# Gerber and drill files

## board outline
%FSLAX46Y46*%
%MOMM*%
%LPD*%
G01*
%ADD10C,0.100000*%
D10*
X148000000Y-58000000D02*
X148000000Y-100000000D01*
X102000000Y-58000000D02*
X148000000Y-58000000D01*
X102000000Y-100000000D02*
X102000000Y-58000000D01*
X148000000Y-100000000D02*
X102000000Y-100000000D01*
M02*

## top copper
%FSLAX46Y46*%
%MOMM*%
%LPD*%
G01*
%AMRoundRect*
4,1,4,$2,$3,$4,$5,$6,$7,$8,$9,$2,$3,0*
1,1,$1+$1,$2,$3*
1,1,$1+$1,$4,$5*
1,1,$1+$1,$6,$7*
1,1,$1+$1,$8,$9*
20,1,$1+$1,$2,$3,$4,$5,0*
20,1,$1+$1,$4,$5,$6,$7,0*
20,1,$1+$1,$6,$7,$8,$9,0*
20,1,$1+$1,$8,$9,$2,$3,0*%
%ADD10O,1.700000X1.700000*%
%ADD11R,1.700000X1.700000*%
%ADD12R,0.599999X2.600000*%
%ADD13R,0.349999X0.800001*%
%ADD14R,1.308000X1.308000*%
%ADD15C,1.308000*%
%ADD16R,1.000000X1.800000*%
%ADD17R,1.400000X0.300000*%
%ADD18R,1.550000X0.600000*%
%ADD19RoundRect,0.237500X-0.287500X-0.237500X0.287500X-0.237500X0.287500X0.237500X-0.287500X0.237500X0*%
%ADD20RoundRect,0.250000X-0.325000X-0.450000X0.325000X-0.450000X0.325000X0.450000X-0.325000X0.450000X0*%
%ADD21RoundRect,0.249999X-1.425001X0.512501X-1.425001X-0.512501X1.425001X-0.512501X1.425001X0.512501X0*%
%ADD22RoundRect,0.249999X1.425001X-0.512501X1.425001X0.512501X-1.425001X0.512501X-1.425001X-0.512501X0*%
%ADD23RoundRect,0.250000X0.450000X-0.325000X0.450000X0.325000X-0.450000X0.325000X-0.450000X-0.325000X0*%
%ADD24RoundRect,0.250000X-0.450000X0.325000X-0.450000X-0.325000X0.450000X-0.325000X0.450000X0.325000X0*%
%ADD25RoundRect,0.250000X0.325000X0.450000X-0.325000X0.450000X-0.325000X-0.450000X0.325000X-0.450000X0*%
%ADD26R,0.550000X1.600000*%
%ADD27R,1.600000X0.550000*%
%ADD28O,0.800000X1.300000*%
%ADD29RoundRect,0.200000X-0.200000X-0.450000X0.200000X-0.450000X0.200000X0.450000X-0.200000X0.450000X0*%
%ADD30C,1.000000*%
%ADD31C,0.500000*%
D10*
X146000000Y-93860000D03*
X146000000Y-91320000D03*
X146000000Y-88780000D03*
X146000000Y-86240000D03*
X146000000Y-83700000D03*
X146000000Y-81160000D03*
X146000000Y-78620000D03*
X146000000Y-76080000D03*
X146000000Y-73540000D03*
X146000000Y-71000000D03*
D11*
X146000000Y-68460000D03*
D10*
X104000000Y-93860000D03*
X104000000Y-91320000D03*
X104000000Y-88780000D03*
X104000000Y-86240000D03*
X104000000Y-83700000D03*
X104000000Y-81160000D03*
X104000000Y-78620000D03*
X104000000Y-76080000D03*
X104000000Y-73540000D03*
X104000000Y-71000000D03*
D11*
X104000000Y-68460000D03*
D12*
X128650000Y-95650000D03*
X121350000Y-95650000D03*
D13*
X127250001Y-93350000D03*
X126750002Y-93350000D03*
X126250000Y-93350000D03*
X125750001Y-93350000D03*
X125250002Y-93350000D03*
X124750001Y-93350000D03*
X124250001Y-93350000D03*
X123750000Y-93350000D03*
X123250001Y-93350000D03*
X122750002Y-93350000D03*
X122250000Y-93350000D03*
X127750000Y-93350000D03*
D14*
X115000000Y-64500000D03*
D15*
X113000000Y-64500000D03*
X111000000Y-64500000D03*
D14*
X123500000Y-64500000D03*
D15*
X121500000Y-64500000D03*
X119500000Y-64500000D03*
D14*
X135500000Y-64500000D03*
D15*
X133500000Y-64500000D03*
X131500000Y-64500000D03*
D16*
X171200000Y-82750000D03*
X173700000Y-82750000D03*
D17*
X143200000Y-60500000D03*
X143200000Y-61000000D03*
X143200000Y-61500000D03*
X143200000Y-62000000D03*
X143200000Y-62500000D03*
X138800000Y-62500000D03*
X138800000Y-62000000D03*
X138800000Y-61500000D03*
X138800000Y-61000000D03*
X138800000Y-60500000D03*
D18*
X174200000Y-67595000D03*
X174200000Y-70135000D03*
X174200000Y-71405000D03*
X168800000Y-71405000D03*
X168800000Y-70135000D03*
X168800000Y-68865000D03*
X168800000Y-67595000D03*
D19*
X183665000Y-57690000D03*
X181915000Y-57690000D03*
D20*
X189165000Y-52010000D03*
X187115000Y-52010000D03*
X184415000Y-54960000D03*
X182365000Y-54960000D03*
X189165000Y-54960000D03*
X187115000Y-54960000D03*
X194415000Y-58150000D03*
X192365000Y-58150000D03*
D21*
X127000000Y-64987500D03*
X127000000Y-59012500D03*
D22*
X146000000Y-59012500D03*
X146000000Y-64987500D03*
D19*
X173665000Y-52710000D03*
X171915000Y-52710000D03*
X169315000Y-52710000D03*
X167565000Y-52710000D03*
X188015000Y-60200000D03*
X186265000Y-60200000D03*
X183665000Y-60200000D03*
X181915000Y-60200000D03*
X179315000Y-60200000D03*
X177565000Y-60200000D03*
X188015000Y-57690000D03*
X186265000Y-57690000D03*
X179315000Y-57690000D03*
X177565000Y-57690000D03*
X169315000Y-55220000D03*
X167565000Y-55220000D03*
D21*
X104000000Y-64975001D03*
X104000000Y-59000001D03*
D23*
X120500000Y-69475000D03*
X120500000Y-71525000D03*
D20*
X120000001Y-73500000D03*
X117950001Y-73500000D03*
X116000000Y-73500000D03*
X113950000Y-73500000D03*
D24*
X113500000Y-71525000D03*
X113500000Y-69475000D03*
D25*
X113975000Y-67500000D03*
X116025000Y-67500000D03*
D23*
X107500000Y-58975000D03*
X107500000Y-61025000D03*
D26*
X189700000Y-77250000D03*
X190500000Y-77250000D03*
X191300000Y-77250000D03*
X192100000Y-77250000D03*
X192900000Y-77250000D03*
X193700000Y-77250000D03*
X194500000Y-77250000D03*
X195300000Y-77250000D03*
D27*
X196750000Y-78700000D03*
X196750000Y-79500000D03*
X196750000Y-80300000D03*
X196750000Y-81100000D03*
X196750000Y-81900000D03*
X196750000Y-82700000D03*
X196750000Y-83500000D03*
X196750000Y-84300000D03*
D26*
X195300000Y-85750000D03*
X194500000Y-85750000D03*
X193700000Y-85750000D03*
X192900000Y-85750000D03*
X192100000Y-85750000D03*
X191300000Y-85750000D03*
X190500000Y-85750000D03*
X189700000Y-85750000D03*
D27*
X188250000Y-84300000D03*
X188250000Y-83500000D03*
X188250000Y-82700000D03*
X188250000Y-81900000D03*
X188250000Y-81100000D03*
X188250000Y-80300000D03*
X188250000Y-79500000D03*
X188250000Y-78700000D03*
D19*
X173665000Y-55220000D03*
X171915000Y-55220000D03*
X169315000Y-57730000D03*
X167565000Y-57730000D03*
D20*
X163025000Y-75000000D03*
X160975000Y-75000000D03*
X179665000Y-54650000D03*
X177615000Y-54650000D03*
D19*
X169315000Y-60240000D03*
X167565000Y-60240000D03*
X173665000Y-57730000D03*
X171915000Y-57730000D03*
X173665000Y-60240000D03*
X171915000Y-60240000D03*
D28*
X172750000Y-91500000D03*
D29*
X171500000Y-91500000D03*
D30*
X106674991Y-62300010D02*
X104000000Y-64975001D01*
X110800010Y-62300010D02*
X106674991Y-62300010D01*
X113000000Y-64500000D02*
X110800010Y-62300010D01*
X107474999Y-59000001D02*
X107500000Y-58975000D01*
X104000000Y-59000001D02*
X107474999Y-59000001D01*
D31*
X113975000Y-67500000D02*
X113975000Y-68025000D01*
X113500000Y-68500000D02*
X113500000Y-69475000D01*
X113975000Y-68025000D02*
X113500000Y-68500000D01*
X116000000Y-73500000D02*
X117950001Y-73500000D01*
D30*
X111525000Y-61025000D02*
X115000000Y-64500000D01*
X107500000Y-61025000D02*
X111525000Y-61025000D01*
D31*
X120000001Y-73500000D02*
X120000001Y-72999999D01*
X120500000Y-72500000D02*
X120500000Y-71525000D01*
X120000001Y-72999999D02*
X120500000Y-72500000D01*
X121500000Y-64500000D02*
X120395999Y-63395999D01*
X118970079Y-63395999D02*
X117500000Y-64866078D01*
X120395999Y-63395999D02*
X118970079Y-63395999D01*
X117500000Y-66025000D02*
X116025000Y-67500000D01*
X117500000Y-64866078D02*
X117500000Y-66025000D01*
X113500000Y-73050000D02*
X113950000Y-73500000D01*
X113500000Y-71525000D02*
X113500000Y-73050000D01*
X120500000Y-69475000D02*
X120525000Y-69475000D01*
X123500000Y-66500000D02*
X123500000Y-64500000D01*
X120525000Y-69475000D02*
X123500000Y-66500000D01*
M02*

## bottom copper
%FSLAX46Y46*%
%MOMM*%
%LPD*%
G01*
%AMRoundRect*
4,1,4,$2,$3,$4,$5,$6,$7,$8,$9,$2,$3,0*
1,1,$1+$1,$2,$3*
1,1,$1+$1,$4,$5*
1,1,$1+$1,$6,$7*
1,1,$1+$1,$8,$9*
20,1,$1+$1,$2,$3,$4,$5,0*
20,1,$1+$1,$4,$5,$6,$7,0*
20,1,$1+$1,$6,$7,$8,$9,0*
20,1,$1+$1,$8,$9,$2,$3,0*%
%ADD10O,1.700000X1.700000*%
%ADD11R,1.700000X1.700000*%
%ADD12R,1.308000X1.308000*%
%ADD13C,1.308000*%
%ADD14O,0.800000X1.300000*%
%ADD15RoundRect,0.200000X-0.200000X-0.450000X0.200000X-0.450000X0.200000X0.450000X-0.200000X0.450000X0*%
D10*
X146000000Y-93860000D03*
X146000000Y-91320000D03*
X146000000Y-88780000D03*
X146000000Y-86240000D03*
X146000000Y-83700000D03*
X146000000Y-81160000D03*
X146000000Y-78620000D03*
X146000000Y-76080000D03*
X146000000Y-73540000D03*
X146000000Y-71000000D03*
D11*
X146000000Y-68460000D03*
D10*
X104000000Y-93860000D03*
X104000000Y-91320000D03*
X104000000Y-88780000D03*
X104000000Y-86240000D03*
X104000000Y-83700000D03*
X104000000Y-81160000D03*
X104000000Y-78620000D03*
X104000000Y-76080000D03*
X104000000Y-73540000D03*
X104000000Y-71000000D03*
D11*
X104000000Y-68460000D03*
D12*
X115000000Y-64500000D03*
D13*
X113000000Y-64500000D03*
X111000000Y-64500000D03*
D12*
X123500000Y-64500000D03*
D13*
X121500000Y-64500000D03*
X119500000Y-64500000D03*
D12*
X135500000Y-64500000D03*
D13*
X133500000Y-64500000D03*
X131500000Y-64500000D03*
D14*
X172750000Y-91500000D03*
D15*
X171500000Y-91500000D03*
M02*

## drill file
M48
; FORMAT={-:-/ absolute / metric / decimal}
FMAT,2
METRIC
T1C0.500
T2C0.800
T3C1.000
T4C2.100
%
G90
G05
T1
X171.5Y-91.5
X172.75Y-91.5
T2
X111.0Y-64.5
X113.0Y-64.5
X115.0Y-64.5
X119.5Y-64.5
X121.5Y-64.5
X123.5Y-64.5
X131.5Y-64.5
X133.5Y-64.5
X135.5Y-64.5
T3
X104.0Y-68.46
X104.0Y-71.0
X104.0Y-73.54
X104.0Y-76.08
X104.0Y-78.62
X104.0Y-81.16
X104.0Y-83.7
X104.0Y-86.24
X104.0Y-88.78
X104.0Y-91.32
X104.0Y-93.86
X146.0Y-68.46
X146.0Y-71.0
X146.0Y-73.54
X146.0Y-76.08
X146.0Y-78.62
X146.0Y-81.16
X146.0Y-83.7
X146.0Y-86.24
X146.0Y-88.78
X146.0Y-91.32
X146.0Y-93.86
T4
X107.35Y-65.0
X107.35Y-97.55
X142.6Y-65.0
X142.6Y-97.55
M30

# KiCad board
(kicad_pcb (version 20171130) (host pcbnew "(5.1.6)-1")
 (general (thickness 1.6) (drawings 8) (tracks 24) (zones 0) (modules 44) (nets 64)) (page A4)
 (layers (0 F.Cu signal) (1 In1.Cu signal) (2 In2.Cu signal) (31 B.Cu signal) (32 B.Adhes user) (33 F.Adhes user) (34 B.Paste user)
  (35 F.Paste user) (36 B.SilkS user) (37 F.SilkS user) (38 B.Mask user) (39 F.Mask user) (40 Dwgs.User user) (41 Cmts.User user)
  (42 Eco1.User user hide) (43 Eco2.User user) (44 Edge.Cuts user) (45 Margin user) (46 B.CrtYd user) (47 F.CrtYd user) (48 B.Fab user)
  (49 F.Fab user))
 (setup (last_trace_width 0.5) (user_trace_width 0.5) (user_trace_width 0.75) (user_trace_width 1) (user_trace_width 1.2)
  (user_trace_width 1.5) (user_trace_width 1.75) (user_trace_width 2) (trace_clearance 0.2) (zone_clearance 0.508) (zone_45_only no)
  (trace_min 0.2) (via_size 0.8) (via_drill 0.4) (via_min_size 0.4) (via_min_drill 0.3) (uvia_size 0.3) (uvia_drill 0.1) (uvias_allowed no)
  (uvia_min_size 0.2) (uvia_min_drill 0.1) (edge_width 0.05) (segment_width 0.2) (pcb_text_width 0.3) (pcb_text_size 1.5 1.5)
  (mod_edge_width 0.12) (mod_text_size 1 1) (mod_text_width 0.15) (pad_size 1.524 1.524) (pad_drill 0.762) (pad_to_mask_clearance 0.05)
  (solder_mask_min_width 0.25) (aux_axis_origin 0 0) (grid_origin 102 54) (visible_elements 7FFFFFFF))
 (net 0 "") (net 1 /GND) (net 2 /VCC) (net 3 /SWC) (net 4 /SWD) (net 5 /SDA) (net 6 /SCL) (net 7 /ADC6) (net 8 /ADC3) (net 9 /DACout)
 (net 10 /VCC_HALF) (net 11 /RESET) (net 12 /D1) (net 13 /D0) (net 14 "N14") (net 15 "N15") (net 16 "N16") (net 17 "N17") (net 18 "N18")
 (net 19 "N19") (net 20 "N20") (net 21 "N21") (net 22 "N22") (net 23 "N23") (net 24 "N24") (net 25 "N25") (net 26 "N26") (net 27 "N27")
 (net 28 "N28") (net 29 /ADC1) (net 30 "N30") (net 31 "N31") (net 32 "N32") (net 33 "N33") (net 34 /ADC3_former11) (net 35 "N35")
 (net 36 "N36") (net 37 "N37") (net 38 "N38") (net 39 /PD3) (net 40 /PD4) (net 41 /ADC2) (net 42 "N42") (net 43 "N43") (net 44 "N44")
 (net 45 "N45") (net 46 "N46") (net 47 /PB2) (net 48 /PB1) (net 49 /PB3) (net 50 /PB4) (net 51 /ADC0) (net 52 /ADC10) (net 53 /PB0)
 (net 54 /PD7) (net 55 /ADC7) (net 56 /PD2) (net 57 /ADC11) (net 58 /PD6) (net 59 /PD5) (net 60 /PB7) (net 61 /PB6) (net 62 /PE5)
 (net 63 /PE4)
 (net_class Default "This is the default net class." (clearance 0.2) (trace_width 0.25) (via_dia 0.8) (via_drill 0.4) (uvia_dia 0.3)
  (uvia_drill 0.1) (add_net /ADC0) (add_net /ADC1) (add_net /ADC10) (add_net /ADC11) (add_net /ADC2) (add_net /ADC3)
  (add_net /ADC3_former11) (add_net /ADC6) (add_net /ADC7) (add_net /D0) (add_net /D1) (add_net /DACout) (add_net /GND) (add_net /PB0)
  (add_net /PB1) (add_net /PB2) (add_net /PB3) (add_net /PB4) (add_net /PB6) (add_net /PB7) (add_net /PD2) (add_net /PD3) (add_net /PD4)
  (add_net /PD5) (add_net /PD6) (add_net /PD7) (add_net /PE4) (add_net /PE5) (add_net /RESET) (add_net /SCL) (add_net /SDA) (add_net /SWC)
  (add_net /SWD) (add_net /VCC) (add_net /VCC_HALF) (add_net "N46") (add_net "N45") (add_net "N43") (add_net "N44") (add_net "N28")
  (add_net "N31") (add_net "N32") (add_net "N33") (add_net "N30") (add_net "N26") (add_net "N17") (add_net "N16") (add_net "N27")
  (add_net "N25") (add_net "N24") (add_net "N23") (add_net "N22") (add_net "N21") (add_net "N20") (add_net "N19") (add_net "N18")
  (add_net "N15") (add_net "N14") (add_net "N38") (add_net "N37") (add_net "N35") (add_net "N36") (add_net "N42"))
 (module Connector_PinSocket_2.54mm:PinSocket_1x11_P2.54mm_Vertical (layer F.Cu) (at 146 68.46)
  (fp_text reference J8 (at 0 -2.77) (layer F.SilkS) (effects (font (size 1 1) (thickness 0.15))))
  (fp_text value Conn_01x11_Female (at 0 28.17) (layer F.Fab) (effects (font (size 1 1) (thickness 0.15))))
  (pad 11 thru_hole oval (at 0 25.4) (size 1.7 1.7) (drill 1) (layers *.Cu *.Mask) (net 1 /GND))
  (pad 10 thru_hole oval (at 0 22.86) (size 1.7 1.7) (drill 1) (layers *.Cu *.Mask) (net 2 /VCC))
  (pad 9 thru_hole oval (at 0 20.32) (size 1.7 1.7) (drill 1) (layers *.Cu *.Mask) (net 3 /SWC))
  (pad 8 thru_hole oval (at 0 17.78) (size 1.7 1.7) (drill 1) (layers *.Cu *.Mask) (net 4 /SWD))
  (pad 7 thru_hole oval (at 0 15.24) (size 1.7 1.7) (drill 1) (layers *.Cu *.Mask) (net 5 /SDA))
  (pad 6 thru_hole oval (at 0 12.7) (size 1.7 1.7) (drill 1) (layers *.Cu *.Mask) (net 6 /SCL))
  (pad 5 thru_hole oval (at 0 10.16) (size 1.7 1.7) (drill 1) (layers *.Cu *.Mask) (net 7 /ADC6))
  (pad 4 thru_hole oval (at 0 7.62) (size 1.7 1.7) (drill 1) (layers *.Cu *.Mask) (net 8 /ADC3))
  (pad 3 thru_hole oval (at 0 5.08) (size 1.7 1.7) (drill 1) (layers *.Cu *.Mask) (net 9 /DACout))
  (pad 2 thru_hole oval (at 0 2.54) (size 1.7 1.7) (drill 1) (layers *.Cu *.Mask) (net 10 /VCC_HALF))
  (pad 1 thru_hole rect (at 0 0) (size 1.7 1.7) (drill 1) (layers *.Cu *.Mask) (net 1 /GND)))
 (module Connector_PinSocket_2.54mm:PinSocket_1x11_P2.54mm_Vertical (layer F.Cu) (at 104 68.46)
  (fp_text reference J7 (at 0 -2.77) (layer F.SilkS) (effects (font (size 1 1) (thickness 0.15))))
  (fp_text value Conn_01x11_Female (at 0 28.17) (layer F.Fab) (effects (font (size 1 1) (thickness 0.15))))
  (pad 11 thru_hole oval (at 0 25.4) (size 1.7 1.7) (drill 1) (layers *.Cu *.Mask) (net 1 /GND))
  (pad 10 thru_hole oval (at 0 22.86) (size 1.7 1.7) (drill 1) (layers *.Cu *.Mask) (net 1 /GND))
  (pad 9 thru_hole oval (at 0 20.32) (size 1.7 1.7) (drill 1) (layers *.Cu *.Mask) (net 1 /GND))
  (pad 8 thru_hole oval (at 0 17.78) (size 1.7 1.7) (drill 1) (layers *.Cu *.Mask) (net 1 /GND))
  (pad 7 thru_hole oval (at 0 15.24) (size 1.7 1.7) (drill 1) (layers *.Cu *.Mask) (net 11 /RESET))
  (pad 6 thru_hole oval (at 0 12.7) (size 1.7 1.7) (drill 1) (layers *.Cu *.Mask) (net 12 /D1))
  (pad 5 thru_hole oval (at 0 10.16) (size 1.7 1.7) (drill 1) (layers *.Cu *.Mask) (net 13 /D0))
  (pad 4 thru_hole oval (at 0 7.62) (size 1.7 1.7) (drill 1) (layers *.Cu *.Mask) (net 2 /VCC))
  (pad 3 thru_hole oval (at 0 5.08) (size 1.7 1.7) (drill 1) (layers *.Cu *.Mask) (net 2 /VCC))
  (pad 2 thru_hole oval (at 0 2.54) (size 1.7 1.7) (drill 1) (layers *.Cu *.Mask) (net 2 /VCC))
  (pad 1 thru_hole rect (at 0 0) (size 1.7 1.7) (drill 1) (layers *.Cu *.Mask) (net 2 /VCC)))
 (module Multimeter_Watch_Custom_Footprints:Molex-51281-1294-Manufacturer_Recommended (layer F.Cu) (at 125 94.5)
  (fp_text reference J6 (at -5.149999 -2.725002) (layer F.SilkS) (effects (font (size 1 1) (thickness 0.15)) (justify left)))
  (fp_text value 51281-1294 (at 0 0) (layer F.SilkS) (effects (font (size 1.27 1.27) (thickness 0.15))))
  (pad MP2 smd rect (at 3.65 1.15) (size 0.599999 2.6) (layers F.Cu F.Paste F.Mask) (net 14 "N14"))
  (pad MP1 smd rect (at -3.65 1.15) (size 0.599999 2.6) (layers F.Cu F.Paste F.Mask) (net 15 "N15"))
  (pad 11 smd rect (at 2.250001 -1.15) (size 0.349999 0.800001) (layers F.Cu F.Paste F.Mask) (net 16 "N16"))
  (pad 10 smd rect (at 1.750002 -1.15) (size 0.349999 0.800001) (layers F.Cu F.Paste F.Mask) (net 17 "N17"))
  (pad 9 smd rect (at 1.25 -1.15) (size 0.349999 0.800001) (layers F.Cu F.Paste F.Mask) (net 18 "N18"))
  (pad 8 smd rect (at 0.750001 -1.15) (size 0.349999 0.800001) (layers F.Cu F.Paste F.Mask) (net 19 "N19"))
  (pad 7 smd rect (at 0.250002 -1.15) (size 0.349999 0.800001) (layers F.Cu F.Paste F.Mask) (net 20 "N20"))
  (pad 6 smd rect (at -0.249999 -1.15) (size 0.349999 0.800001) (layers F.Cu F.Paste F.Mask) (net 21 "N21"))
  (pad 5 smd rect (at -0.749999 -1.15) (size 0.349999 0.800001) (layers F.Cu F.Paste F.Mask) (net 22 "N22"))
  (pad 4 smd rect (at -1.25 -1.15) (size 0.349999 0.800001) (layers F.Cu F.Paste F.Mask) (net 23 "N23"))
  (pad 3 smd rect (at -1.749999 -1.15) (size 0.349999 0.800001) (layers F.Cu F.Paste F.Mask) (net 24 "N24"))
  (pad 2 smd rect (at -2.249998 -1.15) (size 0.349999 0.800001) (layers F.Cu F.Paste F.Mask) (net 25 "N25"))
  (pad 1 smd rect (at -2.75 -1.15) (size 0.349999 0.800001) (layers F.Cu F.Paste F.Mask) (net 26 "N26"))
  (pad 12 smd rect (at 2.75 -1.15) (size 0.349999 0.800001) (layers F.Cu F.Paste F.Mask) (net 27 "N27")))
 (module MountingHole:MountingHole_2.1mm (layer F.Cu) (at 142.6 97.55)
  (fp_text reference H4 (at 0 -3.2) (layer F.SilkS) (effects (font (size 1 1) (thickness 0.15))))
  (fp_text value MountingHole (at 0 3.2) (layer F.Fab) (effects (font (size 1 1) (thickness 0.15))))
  (pad "" np_thru_hole circle (at 0 0) (size 2.1 2.1) (drill 2.1) (layers *.Cu *.Mask)))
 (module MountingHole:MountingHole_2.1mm (layer F.Cu) (at 107.35 97.55)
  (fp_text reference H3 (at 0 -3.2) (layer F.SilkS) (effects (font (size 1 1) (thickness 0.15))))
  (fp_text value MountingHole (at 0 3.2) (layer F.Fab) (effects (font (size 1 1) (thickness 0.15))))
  (pad "" np_thru_hole circle (at 0 0) (size 2.1 2.1) (drill 2.1) (layers *.Cu *.Mask)))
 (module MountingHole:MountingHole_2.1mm (layer F.Cu) (at 142.6 65)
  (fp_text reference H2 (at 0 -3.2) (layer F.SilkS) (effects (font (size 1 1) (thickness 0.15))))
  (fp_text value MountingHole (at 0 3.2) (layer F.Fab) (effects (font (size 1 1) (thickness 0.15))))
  (pad "" np_thru_hole circle (at 0 0) (size 2.1 2.1) (drill 2.1) (layers *.Cu *.Mask)))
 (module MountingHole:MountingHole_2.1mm (layer F.Cu) (at 107.35 65)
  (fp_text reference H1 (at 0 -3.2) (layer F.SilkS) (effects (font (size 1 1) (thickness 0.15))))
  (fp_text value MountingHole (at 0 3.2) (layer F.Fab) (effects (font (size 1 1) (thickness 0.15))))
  (pad "" np_thru_hole circle (at 0 0) (size 2.1 2.1) (drill 2.1) (layers *.Cu *.Mask)))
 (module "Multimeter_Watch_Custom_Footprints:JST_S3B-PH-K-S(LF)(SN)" (layer F.Cu) (at 115 64.5 180)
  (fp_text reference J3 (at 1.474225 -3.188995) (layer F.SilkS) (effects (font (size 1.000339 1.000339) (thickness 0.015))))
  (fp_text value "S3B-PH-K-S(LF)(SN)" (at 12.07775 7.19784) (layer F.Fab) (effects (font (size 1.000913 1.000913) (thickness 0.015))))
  (pad 1 thru_hole rect (at 0 0 180) (size 1.308 1.308) (drill 0.8) (layers *.Cu *.Mask) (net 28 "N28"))
  (pad 2 thru_hole circle (at 2 0 180) (size 1.308 1.308) (drill 0.8) (layers *.Cu *.Mask) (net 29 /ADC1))
  (pad 3 thru_hole circle (at 4 0 180) (size 1.308 1.308) (drill 0.8) (layers *.Cu *.Mask) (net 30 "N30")))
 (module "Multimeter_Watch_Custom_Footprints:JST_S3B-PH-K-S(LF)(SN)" (layer F.Cu) (at 123.5 64.5 180)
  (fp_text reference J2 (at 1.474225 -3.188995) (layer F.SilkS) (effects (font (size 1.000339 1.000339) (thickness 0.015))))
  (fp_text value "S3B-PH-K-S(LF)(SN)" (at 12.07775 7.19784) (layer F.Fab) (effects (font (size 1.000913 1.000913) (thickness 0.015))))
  (pad 1 thru_hole rect (at 0 0 180) (size 1.308 1.308) (drill 0.8) (layers *.Cu *.Mask) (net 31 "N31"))
  (pad 2 thru_hole circle (at 2 0 180) (size 1.308 1.308) (drill 0.8) (layers *.Cu *.Mask) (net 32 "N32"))
  (pad 3 thru_hole circle (at 4 0 180) (size 1.308 1.308) (drill 0.8) (layers *.Cu *.Mask) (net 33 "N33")))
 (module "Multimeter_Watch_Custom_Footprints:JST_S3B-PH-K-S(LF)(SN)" (layer F.Cu) (at 135.5 64.5 180)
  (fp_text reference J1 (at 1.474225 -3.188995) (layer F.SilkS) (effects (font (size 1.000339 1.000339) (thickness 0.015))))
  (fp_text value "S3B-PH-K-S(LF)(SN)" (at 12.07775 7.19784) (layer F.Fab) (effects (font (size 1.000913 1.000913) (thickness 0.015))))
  (pad 1 thru_hole rect (at 0 0 180) (size 1.308 1.308) (drill 0.8) (layers *.Cu *.Mask) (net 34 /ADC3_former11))
  (pad 2 thru_hole circle (at 2 0 180) (size 1.308 1.308) (drill 0.8) (layers *.Cu *.Mask) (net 7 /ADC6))
  (pad 3 thru_hole circle (at 4 0 180) (size 1.308 1.308) (drill 0.8) (layers *.Cu *.Mask) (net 9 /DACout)))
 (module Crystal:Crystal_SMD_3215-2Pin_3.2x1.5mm (layer F.Cu) (at 172.45 82.75)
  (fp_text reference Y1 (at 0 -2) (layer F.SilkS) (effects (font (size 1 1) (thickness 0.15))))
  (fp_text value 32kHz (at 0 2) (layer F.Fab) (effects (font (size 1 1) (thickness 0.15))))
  (pad 2 smd rect (at -1.25 0) (size 1 1.8) (layers F.Cu F.Paste F.Mask) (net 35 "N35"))
  (pad 1 smd rect (at 1.25 0) (size 1 1.8) (layers F.Cu F.Paste F.Mask) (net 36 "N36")))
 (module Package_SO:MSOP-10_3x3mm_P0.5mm (layer F.Cu) (at 141 61.5)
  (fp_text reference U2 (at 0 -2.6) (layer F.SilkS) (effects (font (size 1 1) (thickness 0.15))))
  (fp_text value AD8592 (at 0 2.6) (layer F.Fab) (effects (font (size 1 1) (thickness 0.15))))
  (pad 10 smd rect (at 2.2 -1) (size 1.4 0.3) (layers F.Cu F.Paste F.Mask) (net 2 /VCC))
  (pad 9 smd rect (at 2.2 -0.5) (size 1.4 0.3) (layers F.Cu F.Paste F.Mask) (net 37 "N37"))
  (pad 8 smd rect (at 2.2 0) (size 1.4 0.3) (layers F.Cu F.Paste F.Mask) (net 10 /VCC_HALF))
  (pad 7 smd rect (at 2.2 0.5) (size 1.4 0.3) (layers F.Cu F.Paste F.Mask) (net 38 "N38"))
  (pad 6 smd rect (at 2.2 1) (size 1.4 0.3) (layers F.Cu F.Paste F.Mask) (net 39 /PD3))
  (pad 5 smd rect (at -2.2 1) (size 1.4 0.3) (layers F.Cu F.Paste F.Mask) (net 39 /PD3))
  (pad 4 smd rect (at -2.2 0.5) (size 1.4 0.3) (layers F.Cu F.Paste F.Mask) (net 1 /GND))
  (pad 3 smd rect (at -2.2 0) (size 1.4 0.3) (layers F.Cu F.Paste F.Mask) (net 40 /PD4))
  (pad 2 smd rect (at -2.2 -0.5) (size 1.4 0.3) (layers F.Cu F.Paste F.Mask) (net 9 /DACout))
  (pad 1 smd rect (at -2.2 -1) (size 1.4 0.3) (layers F.Cu F.Paste F.Mask) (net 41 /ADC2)))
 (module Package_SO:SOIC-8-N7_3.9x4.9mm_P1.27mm (layer F.Cu) (at 171.5 69.5)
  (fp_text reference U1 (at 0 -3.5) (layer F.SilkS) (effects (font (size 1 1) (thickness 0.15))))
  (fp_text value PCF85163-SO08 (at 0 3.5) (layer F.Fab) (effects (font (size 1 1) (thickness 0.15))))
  (pad 8 smd rect (at 2.7 -1.905) (size 1.55 0.6) (layers F.Cu F.Paste F.Mask) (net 2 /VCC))
  (pad 6 smd rect (at 2.7 0.635) (size 1.55 0.6) (layers F.Cu F.Paste F.Mask) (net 6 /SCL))
  (pad 5 smd rect (at 2.7 1.905) (size 1.55 0.6) (layers F.Cu F.Paste F.Mask) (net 5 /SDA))
  (pad 4 smd rect (at -2.7 1.905) (size 1.55 0.6) (layers F.Cu F.Paste F.Mask) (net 1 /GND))
  (pad 3 smd rect (at -2.7 0.635) (size 1.55 0.6) (layers F.Cu F.Paste F.Mask) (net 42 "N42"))
  (pad 2 smd rect (at -2.7 -0.635) (size 1.55 0.6) (layers F.Cu F.Paste F.Mask) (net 36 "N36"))
  (pad 1 smd rect (at -2.7 -1.905) (size 1.55 0.6) (layers F.Cu F.Paste F.Mask) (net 35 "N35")))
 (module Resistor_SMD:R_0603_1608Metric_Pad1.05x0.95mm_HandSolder (layer F.Cu) (at 182.79 57.69)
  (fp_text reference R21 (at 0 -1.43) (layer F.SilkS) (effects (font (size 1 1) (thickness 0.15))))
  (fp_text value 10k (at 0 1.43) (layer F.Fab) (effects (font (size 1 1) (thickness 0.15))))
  (pad 2 smd roundrect (at 0.875 0) (size 1.05 0.95) (layers F.Cu F.Paste F.Mask) (roundrect_rratio 0.25) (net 11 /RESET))
  (pad 1 smd roundrect (at -0.875 0) (size 1.05 0.95) (layers F.Cu F.Paste F.Mask) (roundrect_rratio 0.25) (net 2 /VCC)))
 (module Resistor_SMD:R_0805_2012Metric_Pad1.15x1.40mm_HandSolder (layer F.Cu) (at 188.14 52.01)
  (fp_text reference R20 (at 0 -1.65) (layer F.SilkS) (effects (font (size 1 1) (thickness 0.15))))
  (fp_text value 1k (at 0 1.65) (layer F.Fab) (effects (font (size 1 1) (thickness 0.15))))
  (pad 2 smd roundrect (at 1.025 0) (size 1.15 1.4) (layers F.Cu F.Paste F.Mask) (roundrect_rratio 0.217391) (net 13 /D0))
  (pad 1 smd roundrect (at -1.025 0) (size 1.15 1.4) (layers F.Cu F.Paste F.Mask) (roundrect_rratio 0.217391) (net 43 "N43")))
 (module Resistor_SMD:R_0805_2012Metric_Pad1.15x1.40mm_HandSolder (layer F.Cu) (at 183.39 54.96)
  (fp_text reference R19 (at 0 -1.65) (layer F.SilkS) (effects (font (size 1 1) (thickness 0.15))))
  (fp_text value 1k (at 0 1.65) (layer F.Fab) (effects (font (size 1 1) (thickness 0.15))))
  (pad 2 smd roundrect (at 1.025 0) (size 1.15 1.4) (layers F.Cu F.Paste F.Mask) (roundrect_rratio 0.217391) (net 12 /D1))
  (pad 1 smd roundrect (at -1.025 0) (size 1.15 1.4) (layers F.Cu F.Paste F.Mask) (roundrect_rratio 0.217391) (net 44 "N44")))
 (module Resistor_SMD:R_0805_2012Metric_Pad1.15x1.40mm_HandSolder (layer F.Cu) (at 188.14 54.96)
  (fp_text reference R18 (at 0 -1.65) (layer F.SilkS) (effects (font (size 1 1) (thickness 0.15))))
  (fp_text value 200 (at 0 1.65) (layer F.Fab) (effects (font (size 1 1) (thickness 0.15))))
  (pad 2 smd roundrect (at 1.025 0) (size 1.15 1.4) (layers F.Cu F.Paste F.Mask) (roundrect_rratio 0.217391) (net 37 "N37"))
  (pad 1 smd roundrect (at -1.025 0) (size 1.15 1.4) (layers F.Cu F.Paste F.Mask) (roundrect_rratio 0.217391) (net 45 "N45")))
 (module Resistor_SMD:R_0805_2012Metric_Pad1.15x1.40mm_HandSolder (layer F.Cu) (at 193.39 58.15)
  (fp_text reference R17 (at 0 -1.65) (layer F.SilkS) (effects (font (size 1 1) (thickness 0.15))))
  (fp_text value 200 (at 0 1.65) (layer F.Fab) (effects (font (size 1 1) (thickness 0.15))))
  (pad 2 smd roundrect (at 1.025 0) (size 1.15 1.4) (layers F.Cu F.Paste F.Mask) (roundrect_rratio 0.217391) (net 41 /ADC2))
  (pad 1 smd roundrect (at -1.025 0) (size 1.15 1.4) (layers F.Cu F.Paste F.Mask) (roundrect_rratio 0.217391) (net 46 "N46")))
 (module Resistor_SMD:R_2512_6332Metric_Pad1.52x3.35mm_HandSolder (layer F.Cu) (at 127 62 270)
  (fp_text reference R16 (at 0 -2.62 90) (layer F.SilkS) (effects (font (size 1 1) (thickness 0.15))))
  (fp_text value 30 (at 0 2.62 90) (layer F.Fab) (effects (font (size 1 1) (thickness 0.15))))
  (pad 2 smd roundrect (at 2.9875 0 270) (size 1.525 3.35) (layers F.Cu F.Paste F.Mask) (roundrect_rratio 0.163934) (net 37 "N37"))
  (pad 1 smd roundrect (at -2.9875 0 270) (size 1.525 3.35) (layers F.Cu F.Paste F.Mask) (roundrect_rratio 0.163934) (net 10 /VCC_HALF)))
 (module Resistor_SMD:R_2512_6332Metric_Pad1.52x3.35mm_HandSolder (layer F.Cu) (at 146 62 90)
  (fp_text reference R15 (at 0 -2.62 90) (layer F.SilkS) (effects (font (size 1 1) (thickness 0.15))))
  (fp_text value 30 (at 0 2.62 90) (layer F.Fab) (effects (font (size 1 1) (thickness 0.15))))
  (pad 2 smd roundrect (at 2.9875 0 90) (size 1.525 3.35) (layers F.Cu F.Paste F.Mask) (roundrect_rratio 0.163934) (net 41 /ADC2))
  (pad 1 smd roundrect (at -2.9875 0 90) (size 1.525 3.35) (layers F.Cu F.Paste F.Mask) (roundrect_rratio 0.163934) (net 9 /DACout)))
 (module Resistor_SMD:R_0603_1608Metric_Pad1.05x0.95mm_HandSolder (layer F.Cu) (at 172.79 52.71)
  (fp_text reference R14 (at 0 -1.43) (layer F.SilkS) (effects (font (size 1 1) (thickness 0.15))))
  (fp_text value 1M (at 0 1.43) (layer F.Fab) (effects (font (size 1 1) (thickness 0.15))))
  (pad 2 smd roundrect (at 0.875 0) (size 1.05 0.95) (layers F.Cu F.Paste F.Mask) (roundrect_rratio 0.25) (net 1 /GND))
  (pad 1 smd roundrect (at -0.875 0) (size 1.05 0.95) (layers F.Cu F.Paste F.Mask) (roundrect_rratio 0.25) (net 38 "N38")))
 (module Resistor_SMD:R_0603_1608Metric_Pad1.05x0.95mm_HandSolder (layer F.Cu) (at 168.44 52.71)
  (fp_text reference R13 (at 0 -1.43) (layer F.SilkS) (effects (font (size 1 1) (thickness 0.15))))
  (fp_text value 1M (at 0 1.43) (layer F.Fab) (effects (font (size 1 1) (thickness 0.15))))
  (pad 2 smd roundrect (at 0.875 0) (size 1.05 0.95) (layers F.Cu F.Paste F.Mask) (roundrect_rratio 0.25) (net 38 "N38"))
  (pad 1 smd roundrect (at -0.875 0) (size 1.05 0.95) (layers F.Cu F.Paste F.Mask) (roundrect_rratio 0.25) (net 2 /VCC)))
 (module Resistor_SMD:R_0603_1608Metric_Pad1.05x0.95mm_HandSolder (layer F.Cu) (at 187.14 60.2)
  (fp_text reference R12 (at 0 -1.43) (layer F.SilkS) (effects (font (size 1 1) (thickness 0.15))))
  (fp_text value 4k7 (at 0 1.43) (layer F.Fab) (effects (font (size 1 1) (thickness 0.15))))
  (pad 2 smd roundrect (at 0.875 0) (size 1.05 0.95) (layers F.Cu F.Paste F.Mask) (roundrect_rratio 0.25) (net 5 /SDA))
  (pad 1 smd roundrect (at -0.875 0) (size 1.05 0.95) (layers F.Cu F.Paste F.Mask) (roundrect_rratio 0.25) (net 39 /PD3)))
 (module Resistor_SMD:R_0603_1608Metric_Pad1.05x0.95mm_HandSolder (layer F.Cu) (at 182.79 60.2)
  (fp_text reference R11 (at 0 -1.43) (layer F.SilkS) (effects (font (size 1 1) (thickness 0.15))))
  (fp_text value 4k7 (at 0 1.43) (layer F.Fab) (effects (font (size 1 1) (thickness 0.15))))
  (pad 2 smd roundrect (at 0.875 0) (size 1.05 0.95) (layers F.Cu F.Paste F.Mask) (roundrect_rratio 0.25) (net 6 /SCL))
  (pad 1 smd roundrect (at -0.875 0) (size 1.05 0.95) (layers F.Cu F.Paste F.Mask) (roundrect_rratio 0.25) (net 39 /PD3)))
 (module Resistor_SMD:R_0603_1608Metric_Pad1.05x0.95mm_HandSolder (layer F.Cu) (at 178.44 60.2)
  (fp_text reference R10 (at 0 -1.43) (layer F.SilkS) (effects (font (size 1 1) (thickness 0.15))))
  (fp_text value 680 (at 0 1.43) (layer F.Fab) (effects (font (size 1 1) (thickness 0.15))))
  (pad 2 smd roundrect (at 0.875 0) (size 1.05 0.95) (layers F.Cu F.Paste F.Mask) (roundrect_rratio 0.25) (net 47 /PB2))
  (pad 1 smd roundrect (at -0.875 0) (size 1.05 0.95) (layers F.Cu F.Paste F.Mask) (roundrect_rratio 0.25) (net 7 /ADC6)))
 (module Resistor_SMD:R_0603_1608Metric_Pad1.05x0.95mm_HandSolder (layer F.Cu) (at 187.14 57.69)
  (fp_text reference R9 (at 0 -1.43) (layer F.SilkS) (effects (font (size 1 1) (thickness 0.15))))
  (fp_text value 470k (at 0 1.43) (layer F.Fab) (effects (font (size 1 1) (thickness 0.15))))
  (pad 2 smd roundrect (at 0.875 0) (size 1.05 0.95) (layers F.Cu F.Paste F.Mask) (roundrect_rratio 0.25) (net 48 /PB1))
  (pad 1 smd roundrect (at -0.875 0) (size 1.05 0.95) (layers F.Cu F.Paste F.Mask) (roundrect_rratio 0.25) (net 7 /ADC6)))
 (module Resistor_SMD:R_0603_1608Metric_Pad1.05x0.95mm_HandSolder (layer F.Cu) (at 178.44 57.69)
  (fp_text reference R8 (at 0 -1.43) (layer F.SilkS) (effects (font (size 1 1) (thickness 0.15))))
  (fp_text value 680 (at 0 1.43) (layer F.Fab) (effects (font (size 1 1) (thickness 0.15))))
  (pad 2 smd roundrect (at 0.875 0) (size 1.05 0.95) (layers F.Cu F.Paste F.Mask) (roundrect_rratio 0.25) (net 34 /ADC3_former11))
  (pad 1 smd roundrect (at -0.875 0) (size 1.05 0.95) (layers F.Cu F.Paste F.Mask) (roundrect_rratio 0.25) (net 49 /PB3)))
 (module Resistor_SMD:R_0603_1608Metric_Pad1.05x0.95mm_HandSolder (layer F.Cu) (at 168.44 55.22)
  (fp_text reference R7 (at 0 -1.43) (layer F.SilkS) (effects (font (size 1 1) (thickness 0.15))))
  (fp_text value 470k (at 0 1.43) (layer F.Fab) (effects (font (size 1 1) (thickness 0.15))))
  (pad 2 smd roundrect (at 0.875 0) (size 1.05 0.95) (layers F.Cu F.Paste F.Mask) (roundrect_rratio 0.25) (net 34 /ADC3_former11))
  (pad 1 smd roundrect (at -0.875 0) (size 1.05 0.95) (layers F.Cu F.Paste F.Mask) (roundrect_rratio 0.25) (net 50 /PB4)))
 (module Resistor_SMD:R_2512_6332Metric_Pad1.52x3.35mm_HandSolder (layer F.Cu) (at 104 61.987501 270)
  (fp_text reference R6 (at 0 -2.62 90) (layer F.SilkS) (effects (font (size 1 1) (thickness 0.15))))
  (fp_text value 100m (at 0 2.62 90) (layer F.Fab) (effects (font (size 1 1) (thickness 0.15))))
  (pad 2 smd roundrect (at 2.9875 0 270) (size 1.525 3.35) (layers F.Cu F.Paste F.Mask) (roundrect_rratio 0.163934) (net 29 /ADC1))
  (pad 1 smd roundrect (at -2.9875 0 270) (size 1.525 3.35) (layers F.Cu F.Paste F.Mask) (roundrect_rratio 0.163934) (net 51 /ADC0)))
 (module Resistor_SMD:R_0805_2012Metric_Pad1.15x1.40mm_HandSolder (layer F.Cu) (at 120.5 70.5 90)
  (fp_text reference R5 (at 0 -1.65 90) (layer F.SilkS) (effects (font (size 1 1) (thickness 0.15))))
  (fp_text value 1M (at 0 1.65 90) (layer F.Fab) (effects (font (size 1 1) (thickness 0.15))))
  (pad 2 smd roundrect (at 1.025 0 90) (size 1.15 1.4) (layers F.Cu F.Paste F.Mask) (roundrect_rratio 0.217391) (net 31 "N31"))
  (pad 1 smd roundrect (at -1.025 0 90) (size 1.15 1.4) (layers F.Cu F.Paste F.Mask) (roundrect_rratio 0.217391) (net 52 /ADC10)))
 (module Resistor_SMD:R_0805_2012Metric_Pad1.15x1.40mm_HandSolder (layer F.Cu) (at 118.975001 73.5)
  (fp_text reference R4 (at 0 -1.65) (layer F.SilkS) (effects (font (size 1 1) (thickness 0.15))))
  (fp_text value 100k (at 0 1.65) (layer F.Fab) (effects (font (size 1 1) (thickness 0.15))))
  (pad 2 smd roundrect (at 1.025 0) (size 1.15 1.4) (layers F.Cu F.Paste F.Mask) (roundrect_rratio 0.217391) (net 52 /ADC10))
  (pad 1 smd roundrect (at -1.025 0) (size 1.15 1.4) (layers F.Cu F.Paste F.Mask) (roundrect_rratio 0.217391) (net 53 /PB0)))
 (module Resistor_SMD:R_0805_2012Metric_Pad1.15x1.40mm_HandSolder (layer F.Cu) (at 114.975 73.5)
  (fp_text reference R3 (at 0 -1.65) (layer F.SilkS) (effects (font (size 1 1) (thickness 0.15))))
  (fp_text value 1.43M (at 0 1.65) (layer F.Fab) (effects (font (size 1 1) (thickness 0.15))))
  (pad 2 smd roundrect (at 1.025 0) (size 1.15 1.4) (layers F.Cu F.Paste F.Mask) (roundrect_rratio 0.217391) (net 53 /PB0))
  (pad 1 smd roundrect (at -1.025 0) (size 1.15 1.4) (layers F.Cu F.Paste F.Mask) (roundrect_rratio 0.217391) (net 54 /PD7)))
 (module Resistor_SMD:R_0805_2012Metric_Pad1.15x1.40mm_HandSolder (layer F.Cu) (at 113.5 70.5 270)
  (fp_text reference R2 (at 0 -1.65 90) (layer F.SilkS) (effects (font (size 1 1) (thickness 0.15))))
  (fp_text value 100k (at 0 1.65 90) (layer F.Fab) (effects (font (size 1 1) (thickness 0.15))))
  (pad 2 smd roundrect (at 1.025 0 270) (size 1.15 1.4) (layers F.Cu F.Paste F.Mask) (roundrect_rratio 0.217391) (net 54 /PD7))
  (pad 1 smd roundrect (at -1.025 0 270) (size 1.15 1.4) (layers F.Cu F.Paste F.Mask) (roundrect_rratio 0.217391) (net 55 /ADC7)))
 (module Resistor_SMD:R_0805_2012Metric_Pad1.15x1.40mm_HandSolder (layer F.Cu) (at 115 67.5 180)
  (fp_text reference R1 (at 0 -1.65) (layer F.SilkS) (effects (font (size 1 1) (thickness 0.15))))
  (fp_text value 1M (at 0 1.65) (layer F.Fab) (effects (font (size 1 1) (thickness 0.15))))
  (pad 2 smd roundrect (at 1.025 0 180) (size 1.15 1.4) (layers F.Cu F.Paste F.Mask) (roundrect_rratio 0.217391) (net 55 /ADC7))
  (pad 1 smd roundrect (at -1.025 0 180) (size 1.15 1.4) (layers F.Cu F.Paste F.Mask) (roundrect_rratio 0.217391) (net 32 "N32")))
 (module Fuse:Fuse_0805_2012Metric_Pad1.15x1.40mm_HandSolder (layer F.Cu) (at 107.5 60 90)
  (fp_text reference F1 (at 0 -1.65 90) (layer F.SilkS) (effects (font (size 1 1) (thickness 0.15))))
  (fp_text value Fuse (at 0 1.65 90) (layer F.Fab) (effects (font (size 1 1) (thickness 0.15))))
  (pad 2 smd roundrect (at 1.025 0 90) (size 1.15 1.4) (layers F.Cu F.Paste F.Mask) (roundrect_rratio 0.217391) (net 51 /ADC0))
  (pad 1 smd roundrect (at -1.025 0 90) (size 1.15 1.4) (layers F.Cu F.Paste F.Mask) (roundrect_rratio 0.217391) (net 28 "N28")))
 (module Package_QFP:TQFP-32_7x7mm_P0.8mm (layer F.Cu) (at 192.5 81.5)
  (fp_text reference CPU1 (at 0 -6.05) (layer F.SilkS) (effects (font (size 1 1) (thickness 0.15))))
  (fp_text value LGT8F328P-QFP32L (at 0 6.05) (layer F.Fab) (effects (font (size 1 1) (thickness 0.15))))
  (pad 32 smd rect (at -2.8 -4.25 90) (size 1.6 0.55) (layers F.Cu F.Paste F.Mask) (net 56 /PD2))
  (pad 31 smd rect (at -2 -4.25 90) (size 1.6 0.55) (layers F.Cu F.Paste F.Mask) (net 44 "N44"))
  (pad 30 smd rect (at -1.2 -4.25 90) (size 1.6 0.55) (layers F.Cu F.Paste F.Mask) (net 43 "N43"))
  (pad 29 smd rect (at -0.4 -4.25 90) (size 1.6 0.55) (layers F.Cu F.Paste F.Mask) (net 11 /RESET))
  (pad 28 smd rect (at 0.4 -4.25 90) (size 1.6 0.55) (layers F.Cu F.Paste F.Mask) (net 5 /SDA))
  (pad 27 smd rect (at 1.2 -4.25 90) (size 1.6 0.55) (layers F.Cu F.Paste F.Mask) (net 6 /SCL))
  (pad 26 smd rect (at 2 -4.25 90) (size 1.6 0.55) (layers F.Cu F.Paste F.Mask) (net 8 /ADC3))
  (pad 25 smd rect (at 2.8 -4.25 90) (size 1.6 0.55) (layers F.Cu F.Paste F.Mask) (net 41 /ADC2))
  (pad 24 smd rect (at 4.25 -2.8) (size 1.6 0.55) (layers F.Cu F.Paste F.Mask) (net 29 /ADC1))
  (pad 23 smd rect (at 4.25 -2) (size 1.6 0.55) (layers F.Cu F.Paste F.Mask) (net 51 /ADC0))
  (pad 22 smd rect (at 4.25 -1.2) (size 1.6 0.55) (layers F.Cu F.Paste F.Mask) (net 55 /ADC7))
  (pad 21 smd rect (at 4.25 -0.4) (size 1.6 0.55) (layers F.Cu F.Paste F.Mask) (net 4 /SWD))
  (pad 20 smd rect (at 4.25 0.4) (size 1.6 0.55) (layers F.Cu F.Paste F.Mask) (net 52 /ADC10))
  (pad 19 smd rect (at 4.25 1.2) (size 1.6 0.55) (layers F.Cu F.Paste F.Mask) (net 7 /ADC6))
  (pad 18 smd rect (at 4.25 2) (size 1.6 0.55) (layers F.Cu F.Paste F.Mask) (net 3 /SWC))
  (pad 17 smd rect (at 4.25 2.8) (size 1.6 0.55) (layers F.Cu F.Paste F.Mask) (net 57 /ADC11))
  (pad 16 smd rect (at 2.8 4.25 90) (size 1.6 0.55) (layers F.Cu F.Paste F.Mask) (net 50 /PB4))
  (pad 15 smd rect (at 2 4.25 90) (size 1.6 0.55) (layers F.Cu F.Paste F.Mask) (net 49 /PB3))
  (pad 14 smd rect (at 1.2 4.25 90) (size 1.6 0.55) (layers F.Cu F.Paste F.Mask) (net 47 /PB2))
  (pad 13 smd rect (at 0.4 4.25 90) (size 1.6 0.55) (layers F.Cu F.Paste F.Mask) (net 48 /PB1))
  (pad 12 smd rect (at -0.4 4.25 90) (size 1.6 0.55) (layers F.Cu F.Paste F.Mask) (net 53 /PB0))
  (pad 11 smd rect (at -1.2 4.25 90) (size 1.6 0.55) (layers F.Cu F.Paste F.Mask) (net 54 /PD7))
  (pad 10 smd rect (at -2 4.25 90) (size 1.6 0.55) (layers F.Cu F.Paste F.Mask) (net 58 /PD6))
  (pad 9 smd rect (at -2.8 4.25 90) (size 1.6 0.55) (layers F.Cu F.Paste F.Mask) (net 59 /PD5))
  (pad 8 smd rect (at -4.25 2.8) (size 1.6 0.55) (layers F.Cu F.Paste F.Mask) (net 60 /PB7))
  (pad 7 smd rect (at -4.25 2) (size 1.6 0.55) (layers F.Cu F.Paste F.Mask) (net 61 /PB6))
  (pad 6 smd rect (at -4.25 1.2) (size 1.6 0.55) (layers F.Cu F.Paste F.Mask) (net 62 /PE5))
  (pad 5 smd rect (at -4.25 0.4) (size 1.6 0.55) (layers F.Cu F.Paste F.Mask) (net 1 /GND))
  (pad 4 smd rect (at -4.25 -0.4) (size 1.6 0.55) (layers F.Cu F.Paste F.Mask) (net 2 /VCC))
  (pad 3 smd rect (at -4.25 -1.2) (size 1.6 0.55) (layers F.Cu F.Paste F.Mask) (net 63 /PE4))
  (pad 2 smd rect (at -4.25 -2) (size 1.6 0.55) (layers F.Cu F.Paste F.Mask) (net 40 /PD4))
  (pad 1 smd rect (at -4.25 -2.8) (size 1.6 0.55) (layers F.Cu F.Paste F.Mask) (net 39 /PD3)))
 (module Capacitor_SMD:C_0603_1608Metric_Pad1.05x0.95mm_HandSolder (layer F.Cu) (at 172.79 55.22)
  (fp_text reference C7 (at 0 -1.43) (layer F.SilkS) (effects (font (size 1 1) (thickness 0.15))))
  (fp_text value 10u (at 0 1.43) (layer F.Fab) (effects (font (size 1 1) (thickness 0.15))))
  (pad 2 smd roundrect (at 0.875 0) (size 1.05 0.95) (layers F.Cu F.Paste F.Mask) (roundrect_rratio 0.25) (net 1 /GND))
  (pad 1 smd roundrect (at -0.875 0) (size 1.05 0.95) (layers F.Cu F.Paste F.Mask) (roundrect_rratio 0.25) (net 2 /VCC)))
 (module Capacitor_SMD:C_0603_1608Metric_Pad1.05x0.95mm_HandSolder (layer F.Cu) (at 168.44 57.73)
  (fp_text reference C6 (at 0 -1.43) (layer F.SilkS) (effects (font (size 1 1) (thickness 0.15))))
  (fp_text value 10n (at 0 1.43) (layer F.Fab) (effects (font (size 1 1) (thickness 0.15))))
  (pad 2 smd roundrect (at 0.875 0) (size 1.05 0.95) (layers F.Cu F.Paste F.Mask) (roundrect_rratio 0.25) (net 1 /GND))
  (pad 1 smd roundrect (at -0.875 0) (size 1.05 0.95) (layers F.Cu F.Paste F.Mask) (roundrect_rratio 0.25) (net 2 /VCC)))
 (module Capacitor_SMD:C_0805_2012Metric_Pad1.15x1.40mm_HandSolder (layer F.Cu) (at 162 75)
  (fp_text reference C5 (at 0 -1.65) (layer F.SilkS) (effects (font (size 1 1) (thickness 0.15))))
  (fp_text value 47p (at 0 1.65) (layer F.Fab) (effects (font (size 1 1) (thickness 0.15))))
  (pad 2 smd roundrect (at 1.025 0) (size 1.15 1.4) (layers F.Cu F.Paste F.Mask) (roundrect_rratio 0.217391) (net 45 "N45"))
  (pad 1 smd roundrect (at -1.025 0) (size 1.15 1.4) (layers F.Cu F.Paste F.Mask) (roundrect_rratio 0.217391) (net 1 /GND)))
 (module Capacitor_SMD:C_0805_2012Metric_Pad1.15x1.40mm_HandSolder (layer F.Cu) (at 178.64 54.65)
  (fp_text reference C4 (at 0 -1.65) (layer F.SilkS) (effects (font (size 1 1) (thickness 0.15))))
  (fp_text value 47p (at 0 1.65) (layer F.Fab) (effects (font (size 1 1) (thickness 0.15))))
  (pad 2 smd roundrect (at 1.025 0) (size 1.15 1.4) (layers F.Cu F.Paste F.Mask) (roundrect_rratio 0.217391) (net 46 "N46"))
  (pad 1 smd roundrect (at -1.025 0) (size 1.15 1.4) (layers F.Cu F.Paste F.Mask) (roundrect_rratio 0.217391) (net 1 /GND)))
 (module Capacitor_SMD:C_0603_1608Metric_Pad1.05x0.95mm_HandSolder (layer F.Cu) (at 168.44 60.24)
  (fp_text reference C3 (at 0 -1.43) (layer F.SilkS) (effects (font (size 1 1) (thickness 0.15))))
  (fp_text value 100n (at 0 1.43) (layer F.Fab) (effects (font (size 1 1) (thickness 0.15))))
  (pad 2 smd roundrect (at 0.875 0) (size 1.05 0.95) (layers F.Cu F.Paste F.Mask) (roundrect_rratio 0.25) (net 1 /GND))
  (pad 1 smd roundrect (at -0.875 0) (size 1.05 0.95) (layers F.Cu F.Paste F.Mask) (roundrect_rratio 0.25) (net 2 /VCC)))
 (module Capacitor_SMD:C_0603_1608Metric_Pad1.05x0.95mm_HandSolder (layer F.Cu) (at 172.79 57.73)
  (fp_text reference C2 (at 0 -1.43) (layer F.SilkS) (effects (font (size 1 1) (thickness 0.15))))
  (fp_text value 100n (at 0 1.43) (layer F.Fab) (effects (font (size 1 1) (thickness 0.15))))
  (pad 2 smd roundrect (at 0.875 0) (size 1.05 0.95) (layers F.Cu F.Paste F.Mask) (roundrect_rratio 0.25) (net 1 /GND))
  (pad 1 smd roundrect (at -0.875 0) (size 1.05 0.95) (layers F.Cu F.Paste F.Mask) (roundrect_rratio 0.25) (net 2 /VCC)))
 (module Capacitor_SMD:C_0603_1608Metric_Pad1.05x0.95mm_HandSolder (layer F.Cu) (at 172.79 60.24)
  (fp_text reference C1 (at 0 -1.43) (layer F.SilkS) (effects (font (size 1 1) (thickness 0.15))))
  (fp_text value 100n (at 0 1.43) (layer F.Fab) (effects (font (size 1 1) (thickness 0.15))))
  (pad 2 smd roundrect (at 0.875 0) (size 1.05 0.95) (layers F.Cu F.Paste F.Mask) (roundrect_rratio 0.25) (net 2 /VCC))
  (pad 1 smd roundrect (at -0.875 0) (size 1.05 0.95) (layers F.Cu F.Paste F.Mask) (roundrect_rratio 0.25) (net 1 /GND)))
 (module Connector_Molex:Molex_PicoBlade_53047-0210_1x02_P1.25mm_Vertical (layer F.Cu) (at 171.5 91.5)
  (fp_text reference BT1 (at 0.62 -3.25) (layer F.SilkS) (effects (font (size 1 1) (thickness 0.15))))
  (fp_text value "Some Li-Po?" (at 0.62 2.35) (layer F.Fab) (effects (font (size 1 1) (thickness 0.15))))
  (pad 2 thru_hole oval (at 1.25 0) (size 0.8 1.3) (drill 0.5) (layers *.Cu *.Mask) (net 1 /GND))
  (pad 1 thru_hole roundrect (at 0 0) (size 0.8 1.3) (drill 0.5) (layers *.Cu *.Mask) (roundrect_rratio 0.25) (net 2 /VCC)))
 (gr_line (start 148 58) (end 148 100) (layer Edge.Cuts) (width 0.1))
 (gr_line (start 102 58) (end 148 58) (layer Edge.Cuts) (width 0.1))
 (gr_line (start 102 100) (end 102 58) (layer Edge.Cuts) (width 0.1))
 (gr_line (start 148 100) (end 102 100) (layer Edge.Cuts) (width 0.1))
 (segment (start 106.674991 62.30001) (end 104 64.975001) (width 1) (layer F.Cu) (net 29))
 (segment (start 110.80001 62.30001) (end 106.674991 62.30001) (width 1) (layer F.Cu) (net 29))
 (segment (start 113 64.5) (end 110.80001 62.30001) (width 1) (layer F.Cu) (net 29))
 (segment (start 107.474999 59.000001) (end 107.5 58.975) (width 1) (layer F.Cu) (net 51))
 (segment (start 104 59.000001) (end 107.474999 59.000001) (width 1) (layer F.Cu) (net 51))
 (segment (start 113.975 67.5) (end 113.975 68.025) (width 0.5) (layer F.Cu) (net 55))
 (segment (start 113.5 68.5) (end 113.5 69.475) (width 0.5) (layer F.Cu) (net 55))
 (segment (start 113.975 68.025) (end 113.5 68.5) (width 0.5) (layer F.Cu) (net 55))
 (segment (start 116 73.5) (end 117.950001 73.5) (width 0.5) (layer F.Cu) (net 53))
 (segment (start 111.525 61.025) (end 115 64.5) (width 1) (layer F.Cu) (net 28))
 (segment (start 107.5 61.025) (end 111.525 61.025) (width 1) (layer F.Cu) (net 28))
 (segment (start 120.000001 73.5) (end 120.000001 72.999999) (width 0.5) (layer F.Cu) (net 52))
 (segment (start 120.5 72.5) (end 120.5 71.525) (width 0.5) (layer F.Cu) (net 52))
 (segment (start 120.000001 72.999999) (end 120.5 72.5) (width 0.5) (layer F.Cu) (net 52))
 (segment (start 121.5 64.5) (end 120.395999 63.395999) (width 0.5) (layer F.Cu) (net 32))
 (segment (start 118.970079 63.395999) (end 117.5 64.866078) (width 0.5) (layer F.Cu) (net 32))
 (segment (start 120.395999 63.395999) (end 118.970079 63.395999) (width 0.5) (layer F.Cu) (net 32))
 (segment (start 117.5 66.025) (end 116.025 67.5) (width 0.5) (layer F.Cu) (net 32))
 (segment (start 117.5 64.866078) (end 117.5 66.025) (width 0.5) (layer F.Cu) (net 32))
 (segment (start 113.5 73.05) (end 113.95 73.5) (width 0.5) (layer F.Cu) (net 54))
 (segment (start 113.5 71.525) (end 113.5 73.05) (width 0.5) (layer F.Cu) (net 54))
 (segment (start 120.5 69.475) (end 120.525 69.475) (width 0.5) (layer F.Cu) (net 31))
 (segment (start 123.5 66.5) (end 123.5 64.5) (width 0.5) (layer F.Cu) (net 31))
 (segment (start 120.525 69.475) (end 123.5 66.5) (width 0.5) (layer F.Cu) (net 31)))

